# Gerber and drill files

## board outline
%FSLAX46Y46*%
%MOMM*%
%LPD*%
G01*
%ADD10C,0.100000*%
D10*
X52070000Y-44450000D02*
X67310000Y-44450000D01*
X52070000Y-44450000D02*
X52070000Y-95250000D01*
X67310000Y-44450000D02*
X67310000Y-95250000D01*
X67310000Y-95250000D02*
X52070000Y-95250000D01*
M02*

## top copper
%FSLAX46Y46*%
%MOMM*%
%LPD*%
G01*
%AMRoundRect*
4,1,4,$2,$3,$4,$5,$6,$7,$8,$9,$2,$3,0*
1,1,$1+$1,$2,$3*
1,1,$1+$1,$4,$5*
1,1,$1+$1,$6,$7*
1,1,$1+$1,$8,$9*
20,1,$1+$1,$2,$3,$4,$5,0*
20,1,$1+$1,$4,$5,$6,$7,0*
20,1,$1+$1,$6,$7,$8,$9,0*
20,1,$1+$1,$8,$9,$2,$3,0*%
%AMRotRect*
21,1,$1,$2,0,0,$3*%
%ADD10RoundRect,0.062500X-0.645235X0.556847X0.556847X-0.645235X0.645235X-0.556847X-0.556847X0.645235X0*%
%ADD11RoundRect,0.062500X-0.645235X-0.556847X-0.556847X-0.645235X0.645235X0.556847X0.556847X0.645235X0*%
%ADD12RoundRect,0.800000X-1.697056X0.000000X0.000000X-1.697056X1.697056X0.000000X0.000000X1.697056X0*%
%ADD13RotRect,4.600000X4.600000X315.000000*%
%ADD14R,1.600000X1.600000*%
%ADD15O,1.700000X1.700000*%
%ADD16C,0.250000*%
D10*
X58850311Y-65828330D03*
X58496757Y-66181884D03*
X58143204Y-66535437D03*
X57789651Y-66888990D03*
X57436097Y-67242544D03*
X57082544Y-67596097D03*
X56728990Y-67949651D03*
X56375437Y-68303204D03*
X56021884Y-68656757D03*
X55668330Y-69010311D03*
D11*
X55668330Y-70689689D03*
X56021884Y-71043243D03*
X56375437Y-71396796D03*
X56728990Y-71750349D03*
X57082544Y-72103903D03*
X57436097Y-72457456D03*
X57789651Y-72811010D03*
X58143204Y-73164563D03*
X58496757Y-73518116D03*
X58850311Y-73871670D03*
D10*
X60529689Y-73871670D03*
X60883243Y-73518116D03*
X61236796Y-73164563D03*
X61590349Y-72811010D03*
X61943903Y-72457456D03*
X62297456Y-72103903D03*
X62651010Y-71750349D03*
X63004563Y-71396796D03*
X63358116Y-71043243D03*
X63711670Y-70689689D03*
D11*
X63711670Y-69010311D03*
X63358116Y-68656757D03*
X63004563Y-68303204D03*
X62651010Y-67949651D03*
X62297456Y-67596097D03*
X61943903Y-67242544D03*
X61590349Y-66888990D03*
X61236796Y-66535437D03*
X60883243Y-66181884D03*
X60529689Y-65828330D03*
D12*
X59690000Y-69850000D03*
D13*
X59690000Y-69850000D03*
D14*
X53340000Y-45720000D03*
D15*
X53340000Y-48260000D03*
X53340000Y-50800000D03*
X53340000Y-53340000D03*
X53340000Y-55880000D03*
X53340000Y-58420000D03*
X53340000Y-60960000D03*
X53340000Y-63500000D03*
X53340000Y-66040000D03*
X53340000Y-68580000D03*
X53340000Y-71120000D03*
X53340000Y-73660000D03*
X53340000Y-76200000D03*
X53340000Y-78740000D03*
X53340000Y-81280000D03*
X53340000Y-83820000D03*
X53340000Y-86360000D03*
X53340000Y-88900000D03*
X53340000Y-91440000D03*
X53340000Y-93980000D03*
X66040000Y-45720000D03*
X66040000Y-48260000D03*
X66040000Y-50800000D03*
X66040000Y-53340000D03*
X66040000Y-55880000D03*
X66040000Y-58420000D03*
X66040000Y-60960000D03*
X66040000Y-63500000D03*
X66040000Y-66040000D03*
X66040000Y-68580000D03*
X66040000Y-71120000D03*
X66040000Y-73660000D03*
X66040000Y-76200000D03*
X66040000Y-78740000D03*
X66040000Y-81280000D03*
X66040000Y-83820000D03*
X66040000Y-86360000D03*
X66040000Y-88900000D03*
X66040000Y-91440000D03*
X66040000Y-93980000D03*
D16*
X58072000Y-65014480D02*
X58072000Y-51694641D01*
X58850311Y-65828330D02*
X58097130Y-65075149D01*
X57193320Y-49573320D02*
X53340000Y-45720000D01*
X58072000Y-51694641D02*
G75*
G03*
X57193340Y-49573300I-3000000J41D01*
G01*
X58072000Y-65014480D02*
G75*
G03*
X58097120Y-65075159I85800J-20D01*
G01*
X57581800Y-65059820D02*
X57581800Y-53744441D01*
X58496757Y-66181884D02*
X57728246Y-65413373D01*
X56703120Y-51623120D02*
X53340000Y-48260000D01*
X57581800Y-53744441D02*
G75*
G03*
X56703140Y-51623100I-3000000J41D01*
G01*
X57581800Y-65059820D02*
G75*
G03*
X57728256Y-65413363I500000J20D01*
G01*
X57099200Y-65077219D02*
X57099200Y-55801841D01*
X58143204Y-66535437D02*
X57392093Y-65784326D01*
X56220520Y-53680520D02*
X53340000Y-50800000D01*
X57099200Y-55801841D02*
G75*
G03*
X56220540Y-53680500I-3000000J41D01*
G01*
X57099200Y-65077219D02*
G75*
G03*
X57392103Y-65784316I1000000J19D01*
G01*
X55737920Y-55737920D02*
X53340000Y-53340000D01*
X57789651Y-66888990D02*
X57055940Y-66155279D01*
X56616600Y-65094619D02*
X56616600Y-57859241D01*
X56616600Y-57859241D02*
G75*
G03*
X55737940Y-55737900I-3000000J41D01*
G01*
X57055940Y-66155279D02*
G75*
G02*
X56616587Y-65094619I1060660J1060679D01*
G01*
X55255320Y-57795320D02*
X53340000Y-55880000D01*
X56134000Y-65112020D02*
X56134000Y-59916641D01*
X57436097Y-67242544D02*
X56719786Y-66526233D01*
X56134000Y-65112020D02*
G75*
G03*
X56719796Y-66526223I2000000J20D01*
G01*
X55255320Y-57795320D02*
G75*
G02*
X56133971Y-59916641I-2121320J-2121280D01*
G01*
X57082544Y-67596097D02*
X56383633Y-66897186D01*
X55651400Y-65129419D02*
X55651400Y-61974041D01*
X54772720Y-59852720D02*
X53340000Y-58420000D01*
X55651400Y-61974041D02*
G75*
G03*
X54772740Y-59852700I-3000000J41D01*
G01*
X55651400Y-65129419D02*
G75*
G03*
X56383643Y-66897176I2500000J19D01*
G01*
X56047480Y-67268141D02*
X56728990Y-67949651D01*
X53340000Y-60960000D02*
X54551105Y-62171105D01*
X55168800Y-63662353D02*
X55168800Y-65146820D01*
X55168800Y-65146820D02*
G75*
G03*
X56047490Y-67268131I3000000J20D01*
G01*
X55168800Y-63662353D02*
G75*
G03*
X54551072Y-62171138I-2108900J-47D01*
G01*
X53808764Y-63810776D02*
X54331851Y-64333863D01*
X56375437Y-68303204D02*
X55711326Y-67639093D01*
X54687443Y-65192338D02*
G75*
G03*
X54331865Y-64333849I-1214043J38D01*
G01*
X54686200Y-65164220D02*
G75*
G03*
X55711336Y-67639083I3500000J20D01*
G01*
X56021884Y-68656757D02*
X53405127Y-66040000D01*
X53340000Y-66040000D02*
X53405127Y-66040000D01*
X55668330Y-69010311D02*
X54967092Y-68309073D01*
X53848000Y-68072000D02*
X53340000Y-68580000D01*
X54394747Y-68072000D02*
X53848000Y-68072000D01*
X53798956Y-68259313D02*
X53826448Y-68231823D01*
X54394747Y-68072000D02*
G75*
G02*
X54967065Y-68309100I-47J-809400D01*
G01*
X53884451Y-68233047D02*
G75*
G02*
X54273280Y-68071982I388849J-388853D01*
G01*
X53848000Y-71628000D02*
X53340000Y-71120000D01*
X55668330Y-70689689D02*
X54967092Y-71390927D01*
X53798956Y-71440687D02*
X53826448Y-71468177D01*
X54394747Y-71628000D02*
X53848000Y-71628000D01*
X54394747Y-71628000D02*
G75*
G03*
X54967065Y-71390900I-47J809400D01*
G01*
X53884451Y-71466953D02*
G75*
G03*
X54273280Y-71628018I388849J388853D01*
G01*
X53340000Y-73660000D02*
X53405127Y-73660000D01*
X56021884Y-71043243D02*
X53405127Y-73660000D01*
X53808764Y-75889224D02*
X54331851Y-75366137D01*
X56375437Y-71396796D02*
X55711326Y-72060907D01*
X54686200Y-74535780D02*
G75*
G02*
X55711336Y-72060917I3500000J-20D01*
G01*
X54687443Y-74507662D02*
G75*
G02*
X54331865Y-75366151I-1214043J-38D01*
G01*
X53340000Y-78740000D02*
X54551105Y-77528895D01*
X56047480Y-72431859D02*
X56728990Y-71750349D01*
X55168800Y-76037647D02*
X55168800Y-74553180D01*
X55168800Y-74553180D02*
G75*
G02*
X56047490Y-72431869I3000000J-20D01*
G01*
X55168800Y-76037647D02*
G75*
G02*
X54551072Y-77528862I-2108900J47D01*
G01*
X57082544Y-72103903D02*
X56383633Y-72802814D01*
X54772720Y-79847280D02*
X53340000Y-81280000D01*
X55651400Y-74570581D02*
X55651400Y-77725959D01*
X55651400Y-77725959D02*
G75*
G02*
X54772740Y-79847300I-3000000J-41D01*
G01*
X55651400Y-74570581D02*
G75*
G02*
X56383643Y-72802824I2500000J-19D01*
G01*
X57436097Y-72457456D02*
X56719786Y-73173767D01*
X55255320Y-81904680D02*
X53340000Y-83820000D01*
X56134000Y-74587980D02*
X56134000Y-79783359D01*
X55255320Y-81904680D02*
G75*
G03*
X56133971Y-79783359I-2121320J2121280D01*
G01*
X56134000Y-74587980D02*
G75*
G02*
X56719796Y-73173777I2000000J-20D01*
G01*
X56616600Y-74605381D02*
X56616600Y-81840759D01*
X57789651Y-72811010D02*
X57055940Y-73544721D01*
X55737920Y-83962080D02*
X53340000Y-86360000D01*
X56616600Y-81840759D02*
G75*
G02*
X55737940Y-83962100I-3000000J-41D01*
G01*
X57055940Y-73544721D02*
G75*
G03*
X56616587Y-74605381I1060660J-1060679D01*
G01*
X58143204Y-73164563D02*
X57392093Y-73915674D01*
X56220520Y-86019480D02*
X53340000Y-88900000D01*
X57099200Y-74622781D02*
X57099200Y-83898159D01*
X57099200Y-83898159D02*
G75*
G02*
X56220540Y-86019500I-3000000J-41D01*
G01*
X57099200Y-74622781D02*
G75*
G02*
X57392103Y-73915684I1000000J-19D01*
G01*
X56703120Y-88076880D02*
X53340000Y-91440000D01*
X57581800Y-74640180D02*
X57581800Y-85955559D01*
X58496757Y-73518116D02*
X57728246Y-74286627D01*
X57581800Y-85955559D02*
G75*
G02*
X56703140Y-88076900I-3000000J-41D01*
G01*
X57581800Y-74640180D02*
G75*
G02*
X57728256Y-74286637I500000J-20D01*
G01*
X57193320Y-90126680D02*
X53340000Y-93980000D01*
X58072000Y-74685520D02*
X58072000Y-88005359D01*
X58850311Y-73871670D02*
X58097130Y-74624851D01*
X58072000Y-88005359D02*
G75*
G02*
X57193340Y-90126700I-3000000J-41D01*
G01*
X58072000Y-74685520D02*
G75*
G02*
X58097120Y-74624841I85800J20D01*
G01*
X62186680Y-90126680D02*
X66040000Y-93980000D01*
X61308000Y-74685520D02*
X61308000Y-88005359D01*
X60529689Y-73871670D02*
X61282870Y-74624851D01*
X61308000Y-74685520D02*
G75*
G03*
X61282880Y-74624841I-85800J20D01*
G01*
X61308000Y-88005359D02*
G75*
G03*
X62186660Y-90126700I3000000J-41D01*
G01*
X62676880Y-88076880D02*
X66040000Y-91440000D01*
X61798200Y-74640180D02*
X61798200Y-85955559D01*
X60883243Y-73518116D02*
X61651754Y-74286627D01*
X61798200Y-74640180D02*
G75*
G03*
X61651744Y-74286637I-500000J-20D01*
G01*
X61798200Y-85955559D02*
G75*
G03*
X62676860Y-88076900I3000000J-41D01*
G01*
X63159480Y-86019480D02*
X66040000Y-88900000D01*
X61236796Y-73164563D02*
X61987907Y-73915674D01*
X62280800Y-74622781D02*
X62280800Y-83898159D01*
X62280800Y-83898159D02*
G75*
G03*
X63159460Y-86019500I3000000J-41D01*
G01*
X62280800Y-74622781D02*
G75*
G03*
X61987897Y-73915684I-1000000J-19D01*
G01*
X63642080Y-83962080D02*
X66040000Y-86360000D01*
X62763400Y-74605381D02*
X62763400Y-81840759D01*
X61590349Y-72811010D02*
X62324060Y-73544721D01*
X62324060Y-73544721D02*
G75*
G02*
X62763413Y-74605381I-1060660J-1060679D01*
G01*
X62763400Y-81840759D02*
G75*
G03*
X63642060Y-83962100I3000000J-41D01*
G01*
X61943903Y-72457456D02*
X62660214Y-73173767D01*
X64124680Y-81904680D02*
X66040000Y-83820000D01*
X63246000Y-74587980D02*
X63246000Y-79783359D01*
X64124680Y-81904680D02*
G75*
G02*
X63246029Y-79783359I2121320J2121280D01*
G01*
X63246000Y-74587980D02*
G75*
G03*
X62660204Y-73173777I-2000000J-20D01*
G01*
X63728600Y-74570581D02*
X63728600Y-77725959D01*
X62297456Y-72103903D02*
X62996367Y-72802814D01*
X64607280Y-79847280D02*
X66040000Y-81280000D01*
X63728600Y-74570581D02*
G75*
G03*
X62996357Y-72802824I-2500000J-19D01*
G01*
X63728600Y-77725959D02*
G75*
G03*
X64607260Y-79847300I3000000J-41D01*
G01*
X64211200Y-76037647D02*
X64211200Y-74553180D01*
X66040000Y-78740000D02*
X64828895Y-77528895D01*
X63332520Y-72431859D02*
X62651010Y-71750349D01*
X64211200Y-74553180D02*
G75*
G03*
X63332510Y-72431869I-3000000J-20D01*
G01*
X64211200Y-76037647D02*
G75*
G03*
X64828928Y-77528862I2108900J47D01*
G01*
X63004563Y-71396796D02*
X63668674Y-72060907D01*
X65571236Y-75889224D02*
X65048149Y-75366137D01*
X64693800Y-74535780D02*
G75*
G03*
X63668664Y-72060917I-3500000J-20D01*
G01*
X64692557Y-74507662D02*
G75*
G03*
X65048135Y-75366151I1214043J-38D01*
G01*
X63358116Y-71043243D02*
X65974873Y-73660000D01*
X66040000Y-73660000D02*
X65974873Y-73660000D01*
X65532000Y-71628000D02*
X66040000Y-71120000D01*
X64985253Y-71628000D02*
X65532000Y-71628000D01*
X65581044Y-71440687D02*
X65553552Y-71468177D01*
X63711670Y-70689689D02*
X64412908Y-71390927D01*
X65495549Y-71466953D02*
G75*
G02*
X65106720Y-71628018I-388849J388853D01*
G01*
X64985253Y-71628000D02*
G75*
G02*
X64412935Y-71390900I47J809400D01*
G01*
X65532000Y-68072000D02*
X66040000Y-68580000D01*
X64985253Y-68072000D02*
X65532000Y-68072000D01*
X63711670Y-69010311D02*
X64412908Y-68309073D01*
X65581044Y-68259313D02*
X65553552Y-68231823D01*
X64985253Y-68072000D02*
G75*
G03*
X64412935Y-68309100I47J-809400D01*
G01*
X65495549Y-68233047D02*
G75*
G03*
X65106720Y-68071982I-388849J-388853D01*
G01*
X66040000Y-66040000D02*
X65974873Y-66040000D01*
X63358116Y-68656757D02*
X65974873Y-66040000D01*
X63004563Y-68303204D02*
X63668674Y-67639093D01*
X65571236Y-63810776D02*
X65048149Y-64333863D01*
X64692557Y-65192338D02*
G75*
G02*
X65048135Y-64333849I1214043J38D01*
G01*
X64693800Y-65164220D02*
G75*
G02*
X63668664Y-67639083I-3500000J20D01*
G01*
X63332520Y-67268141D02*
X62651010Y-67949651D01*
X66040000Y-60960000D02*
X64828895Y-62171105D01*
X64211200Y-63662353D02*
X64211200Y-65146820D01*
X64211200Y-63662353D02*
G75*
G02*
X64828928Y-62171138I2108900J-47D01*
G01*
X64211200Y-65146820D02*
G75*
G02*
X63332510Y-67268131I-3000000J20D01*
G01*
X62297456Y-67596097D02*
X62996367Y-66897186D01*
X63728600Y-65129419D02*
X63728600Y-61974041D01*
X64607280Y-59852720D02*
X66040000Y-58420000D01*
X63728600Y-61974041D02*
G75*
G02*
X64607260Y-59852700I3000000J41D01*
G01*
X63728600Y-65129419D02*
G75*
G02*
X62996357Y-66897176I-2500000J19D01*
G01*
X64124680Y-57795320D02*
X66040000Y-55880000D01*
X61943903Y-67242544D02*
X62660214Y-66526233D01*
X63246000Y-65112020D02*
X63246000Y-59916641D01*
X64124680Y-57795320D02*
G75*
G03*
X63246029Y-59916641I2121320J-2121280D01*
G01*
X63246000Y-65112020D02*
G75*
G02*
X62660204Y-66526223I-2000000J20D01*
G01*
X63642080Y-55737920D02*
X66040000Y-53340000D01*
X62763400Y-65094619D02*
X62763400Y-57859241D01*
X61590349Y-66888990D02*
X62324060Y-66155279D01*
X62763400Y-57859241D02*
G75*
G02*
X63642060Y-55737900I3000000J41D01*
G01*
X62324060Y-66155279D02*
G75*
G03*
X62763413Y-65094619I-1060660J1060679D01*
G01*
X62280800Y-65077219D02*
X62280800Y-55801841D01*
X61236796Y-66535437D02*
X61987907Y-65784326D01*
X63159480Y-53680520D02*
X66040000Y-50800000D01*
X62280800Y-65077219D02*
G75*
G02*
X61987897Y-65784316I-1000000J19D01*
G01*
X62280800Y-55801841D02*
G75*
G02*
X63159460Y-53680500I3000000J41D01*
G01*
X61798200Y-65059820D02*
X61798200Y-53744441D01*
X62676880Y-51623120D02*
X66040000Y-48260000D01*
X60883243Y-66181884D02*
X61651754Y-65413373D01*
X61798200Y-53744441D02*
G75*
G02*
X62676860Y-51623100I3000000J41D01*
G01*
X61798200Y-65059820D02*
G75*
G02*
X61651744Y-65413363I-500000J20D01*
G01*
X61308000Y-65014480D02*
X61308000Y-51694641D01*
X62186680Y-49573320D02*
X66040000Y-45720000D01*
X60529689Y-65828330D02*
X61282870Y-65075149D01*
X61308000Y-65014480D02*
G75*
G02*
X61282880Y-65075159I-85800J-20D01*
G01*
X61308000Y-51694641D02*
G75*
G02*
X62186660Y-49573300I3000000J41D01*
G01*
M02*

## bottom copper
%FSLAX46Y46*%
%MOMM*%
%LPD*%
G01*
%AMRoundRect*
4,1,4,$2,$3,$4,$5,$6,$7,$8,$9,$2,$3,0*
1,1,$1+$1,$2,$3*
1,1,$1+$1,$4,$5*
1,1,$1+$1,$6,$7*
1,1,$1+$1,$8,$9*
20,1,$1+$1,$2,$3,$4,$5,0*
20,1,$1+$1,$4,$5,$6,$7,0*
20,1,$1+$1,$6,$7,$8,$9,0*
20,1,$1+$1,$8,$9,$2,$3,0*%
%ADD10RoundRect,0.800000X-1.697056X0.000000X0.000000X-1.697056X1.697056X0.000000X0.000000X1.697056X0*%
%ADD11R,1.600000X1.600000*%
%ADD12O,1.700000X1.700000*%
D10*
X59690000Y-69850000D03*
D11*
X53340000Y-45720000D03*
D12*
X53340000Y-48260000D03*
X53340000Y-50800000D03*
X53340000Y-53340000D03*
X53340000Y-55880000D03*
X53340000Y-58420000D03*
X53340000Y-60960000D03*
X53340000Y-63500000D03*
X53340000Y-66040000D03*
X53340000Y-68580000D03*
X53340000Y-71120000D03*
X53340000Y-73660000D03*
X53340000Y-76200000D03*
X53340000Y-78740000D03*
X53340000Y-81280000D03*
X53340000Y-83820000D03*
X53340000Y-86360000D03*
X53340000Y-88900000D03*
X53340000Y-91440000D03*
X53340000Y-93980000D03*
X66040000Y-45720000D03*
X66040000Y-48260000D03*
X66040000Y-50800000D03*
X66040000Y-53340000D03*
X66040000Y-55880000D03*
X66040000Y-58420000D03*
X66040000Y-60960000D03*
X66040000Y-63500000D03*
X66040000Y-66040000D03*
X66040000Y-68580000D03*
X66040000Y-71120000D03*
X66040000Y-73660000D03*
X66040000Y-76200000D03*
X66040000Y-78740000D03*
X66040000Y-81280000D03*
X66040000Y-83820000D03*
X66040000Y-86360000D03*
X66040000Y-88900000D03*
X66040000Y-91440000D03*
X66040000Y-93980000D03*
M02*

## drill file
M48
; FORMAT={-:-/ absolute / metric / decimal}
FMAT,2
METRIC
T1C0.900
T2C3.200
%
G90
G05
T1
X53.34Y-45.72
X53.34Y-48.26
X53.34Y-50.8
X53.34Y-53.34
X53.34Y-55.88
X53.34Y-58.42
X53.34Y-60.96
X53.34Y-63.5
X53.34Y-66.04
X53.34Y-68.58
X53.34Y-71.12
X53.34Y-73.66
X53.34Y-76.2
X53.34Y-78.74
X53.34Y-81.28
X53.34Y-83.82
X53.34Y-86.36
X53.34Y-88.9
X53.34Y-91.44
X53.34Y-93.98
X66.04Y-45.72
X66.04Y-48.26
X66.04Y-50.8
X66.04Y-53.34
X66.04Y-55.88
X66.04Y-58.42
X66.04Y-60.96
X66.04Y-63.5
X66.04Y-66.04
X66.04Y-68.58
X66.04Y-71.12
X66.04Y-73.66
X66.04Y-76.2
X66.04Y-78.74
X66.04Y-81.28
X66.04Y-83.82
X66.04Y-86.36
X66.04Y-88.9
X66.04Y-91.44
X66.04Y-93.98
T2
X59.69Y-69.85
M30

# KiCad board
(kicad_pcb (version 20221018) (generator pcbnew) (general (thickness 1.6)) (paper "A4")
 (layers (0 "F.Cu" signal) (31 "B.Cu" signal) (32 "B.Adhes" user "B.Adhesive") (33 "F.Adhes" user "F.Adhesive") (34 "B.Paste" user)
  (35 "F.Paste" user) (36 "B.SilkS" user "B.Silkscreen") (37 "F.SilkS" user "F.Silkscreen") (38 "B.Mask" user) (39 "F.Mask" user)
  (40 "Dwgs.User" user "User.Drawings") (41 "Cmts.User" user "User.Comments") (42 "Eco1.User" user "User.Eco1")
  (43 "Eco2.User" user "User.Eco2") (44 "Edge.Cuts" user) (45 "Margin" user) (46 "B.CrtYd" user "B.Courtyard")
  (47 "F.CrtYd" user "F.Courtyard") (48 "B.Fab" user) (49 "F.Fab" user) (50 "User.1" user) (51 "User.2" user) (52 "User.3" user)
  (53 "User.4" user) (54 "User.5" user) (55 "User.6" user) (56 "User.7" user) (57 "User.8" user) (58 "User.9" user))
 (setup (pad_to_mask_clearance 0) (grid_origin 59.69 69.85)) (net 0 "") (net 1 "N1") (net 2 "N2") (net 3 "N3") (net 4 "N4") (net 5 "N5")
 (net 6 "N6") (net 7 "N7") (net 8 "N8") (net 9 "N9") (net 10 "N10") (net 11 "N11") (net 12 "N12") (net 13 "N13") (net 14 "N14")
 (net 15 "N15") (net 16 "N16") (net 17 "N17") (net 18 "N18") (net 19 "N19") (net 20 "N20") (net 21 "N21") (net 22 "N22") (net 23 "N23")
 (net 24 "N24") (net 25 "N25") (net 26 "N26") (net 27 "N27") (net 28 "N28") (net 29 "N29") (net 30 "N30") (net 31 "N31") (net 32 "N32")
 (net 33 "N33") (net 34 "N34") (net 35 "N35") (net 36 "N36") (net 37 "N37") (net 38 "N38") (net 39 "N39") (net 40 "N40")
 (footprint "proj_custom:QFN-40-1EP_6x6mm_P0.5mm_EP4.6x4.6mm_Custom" (layer "F.Cu") (at 59.69 69.85 -45)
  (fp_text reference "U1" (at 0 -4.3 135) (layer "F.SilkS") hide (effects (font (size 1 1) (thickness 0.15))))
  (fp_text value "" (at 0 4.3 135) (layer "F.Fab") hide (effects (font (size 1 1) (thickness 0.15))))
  (pad "" smd roundrect (at -1.725 -1.725 315) (size 0.93 0.93) (layers "F.Paste") (roundrect_rratio 0.25))
  (pad "" smd roundrect (at -1.725 -0.575 315) (size 0.93 0.93) (layers "F.Paste") (roundrect_rratio 0.25))
  (pad "" smd roundrect (at -1.725 0.575 315) (size 0.93 0.93) (layers "F.Paste") (roundrect_rratio 0.25))
  (pad "" smd roundrect (at -1.725 1.725 315) (size 0.93 0.93) (layers "F.Paste") (roundrect_rratio 0.25))
  (pad "" smd roundrect (at -0.575 -1.725 315) (size 0.93 0.93) (layers "F.Paste") (roundrect_rratio 0.25))
  (pad "" smd roundrect (at -0.575 -0.575 315) (size 0.93 0.93) (layers "F.Paste") (roundrect_rratio 0.25))
  (pad "" smd roundrect (at -0.575 0.575 315) (size 0.93 0.93) (layers "F.Paste") (roundrect_rratio 0.25))
  (pad "" smd roundrect (at -0.575 1.725 315) (size 0.93 0.93) (layers "F.Paste") (roundrect_rratio 0.25))
  (pad "" smd roundrect (at 0.575 -1.725 315) (size 0.93 0.93) (layers "F.Paste") (roundrect_rratio 0.25))
  (pad "" smd roundrect (at 0.575 -0.575 315) (size 0.93 0.93) (layers "F.Paste") (roundrect_rratio 0.25))
  (pad "" smd roundrect (at 0.575 0.575 315) (size 0.93 0.93) (layers "F.Paste") (roundrect_rratio 0.25))
  (pad "" smd roundrect (at 0.575 1.725 315) (size 0.93 0.93) (layers "F.Paste") (roundrect_rratio 0.25))
  (pad "" smd roundrect (at 1.725 -1.725 315) (size 0.93 0.93) (layers "F.Paste") (roundrect_rratio 0.25))
  (pad "" smd roundrect (at 1.725 -0.575 315) (size 0.93 0.93) (layers "F.Paste") (roundrect_rratio 0.25))
  (pad "" smd roundrect (at 1.725 0.575 315) (size 0.93 0.93) (layers "F.Paste") (roundrect_rratio 0.25))
  (pad "" smd roundrect (at 1.725 1.725 315) (size 0.93 0.93) (layers "F.Paste") (roundrect_rratio 0.25))
  (pad "1" smd roundrect (at -3.4375 -2.25 315) (size 1.825 0.25) (layers "F.Cu" "F.Paste" "F.Mask") (roundrect_rratio 0.25) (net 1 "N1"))
  (pad "2" smd roundrect (at -3.4375 -1.75 315) (size 1.825 0.25) (layers "F.Cu" "F.Paste" "F.Mask") (roundrect_rratio 0.25) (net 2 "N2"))
  (pad "3" smd roundrect (at -3.4375 -1.25 315) (size 1.825 0.25) (layers "F.Cu" "F.Paste" "F.Mask") (roundrect_rratio 0.25) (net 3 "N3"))
  (pad "4" smd roundrect (at -3.4375 -0.75 315) (size 1.825 0.25) (layers "F.Cu" "F.Paste" "F.Mask") (roundrect_rratio 0.25) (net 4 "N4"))
  (pad "5" smd roundrect (at -3.4375 -0.25 315) (size 1.825 0.25) (layers "F.Cu" "F.Paste" "F.Mask") (roundrect_rratio 0.25) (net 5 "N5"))
  (pad "6" smd roundrect (at -3.4375 0.25 315) (size 1.825 0.25) (layers "F.Cu" "F.Paste" "F.Mask") (roundrect_rratio 0.25) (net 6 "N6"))
  (pad "7" smd roundrect (at -3.4375 0.75 315) (size 1.825 0.25) (layers "F.Cu" "F.Paste" "F.Mask") (roundrect_rratio 0.25) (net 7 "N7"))
  (pad "8" smd roundrect (at -3.4375 1.25 315) (size 1.825 0.25) (layers "F.Cu" "F.Paste" "F.Mask") (roundrect_rratio 0.25) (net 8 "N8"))
  (pad "9" smd roundrect (at -3.4375 1.75 315) (size 1.825 0.25) (layers "F.Cu" "F.Paste" "F.Mask") (roundrect_rratio 0.25) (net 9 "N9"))
  (pad "10" smd roundrect (at -3.4375 2.25 315) (size 1.825 0.25) (layers "F.Cu" "F.Paste" "F.Mask") (roundrect_rratio 0.25) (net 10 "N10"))
  (pad "11" smd roundrect (at -2.25 3.4375 315) (size 0.25 1.825) (layers "F.Cu" "F.Paste" "F.Mask") (roundrect_rratio 0.25) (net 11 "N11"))
  (pad "12" smd roundrect (at -1.75 3.4375 315) (size 0.25 1.825) (layers "F.Cu" "F.Paste" "F.Mask") (roundrect_rratio 0.25) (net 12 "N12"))
  (pad "13" smd roundrect (at -1.25 3.4375 315) (size 0.25 1.825) (layers "F.Cu" "F.Paste" "F.Mask") (roundrect_rratio 0.25) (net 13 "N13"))
  (pad "14" smd roundrect (at -0.75 3.4375 315) (size 0.25 1.825) (layers "F.Cu" "F.Paste" "F.Mask") (roundrect_rratio 0.25) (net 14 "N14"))
  (pad "15" smd roundrect (at -0.25 3.4375 315) (size 0.25 1.825) (layers "F.Cu" "F.Paste" "F.Mask") (roundrect_rratio 0.25) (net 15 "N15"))
  (pad "16" smd roundrect (at 0.25 3.4375 315) (size 0.25 1.825) (layers "F.Cu" "F.Paste" "F.Mask") (roundrect_rratio 0.25) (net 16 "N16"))
  (pad "17" smd roundrect (at 0.75 3.4375 315) (size 0.25 1.825) (layers "F.Cu" "F.Paste" "F.Mask") (roundrect_rratio 0.25) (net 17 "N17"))
  (pad "18" smd roundrect (at 1.25 3.4375 315) (size 0.25 1.825) (layers "F.Cu" "F.Paste" "F.Mask") (roundrect_rratio 0.25) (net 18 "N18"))
  (pad "19" smd roundrect (at 1.75 3.4375 315) (size 0.25 1.825) (layers "F.Cu" "F.Paste" "F.Mask") (roundrect_rratio 0.25) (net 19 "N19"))
  (pad "20" smd roundrect (at 2.25 3.4375 315) (size 0.25 1.825) (layers "F.Cu" "F.Paste" "F.Mask") (roundrect_rratio 0.25) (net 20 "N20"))
  (pad "21" smd roundrect (at 3.4375 2.25 315) (size 1.825 0.25) (layers "F.Cu" "F.Paste" "F.Mask") (roundrect_rratio 0.25) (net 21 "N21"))
  (pad "22" smd roundrect (at 3.4375 1.75 315) (size 1.825 0.25) (layers "F.Cu" "F.Paste" "F.Mask") (roundrect_rratio 0.25) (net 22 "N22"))
  (pad "23" smd roundrect (at 3.4375 1.25 315) (size 1.825 0.25) (layers "F.Cu" "F.Paste" "F.Mask") (roundrect_rratio 0.25) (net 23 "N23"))
  (pad "24" smd roundrect (at 3.4375 0.75 315) (size 1.825 0.25) (layers "F.Cu" "F.Paste" "F.Mask") (roundrect_rratio 0.25) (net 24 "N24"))
  (pad "25" smd roundrect (at 3.4375 0.25 315) (size 1.825 0.25) (layers "F.Cu" "F.Paste" "F.Mask") (roundrect_rratio 0.25) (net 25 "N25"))
  (pad "26" smd roundrect (at 3.4375 -0.25 315) (size 1.825 0.25) (layers "F.Cu" "F.Paste" "F.Mask") (roundrect_rratio 0.25) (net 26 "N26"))
  (pad "27" smd roundrect (at 3.4375 -0.75 315) (size 1.825 0.25) (layers "F.Cu" "F.Paste" "F.Mask") (roundrect_rratio 0.25) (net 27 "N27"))
  (pad "28" smd roundrect (at 3.4375 -1.25 315) (size 1.825 0.25) (layers "F.Cu" "F.Paste" "F.Mask") (roundrect_rratio 0.25) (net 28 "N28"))
  (pad "29" smd roundrect (at 3.4375 -1.75 315) (size 1.825 0.25) (layers "F.Cu" "F.Paste" "F.Mask") (roundrect_rratio 0.25) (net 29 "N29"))
  (pad "30" smd roundrect (at 3.4375 -2.25 315) (size 1.825 0.25) (layers "F.Cu" "F.Paste" "F.Mask") (roundrect_rratio 0.25) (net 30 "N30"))
  (pad "31" smd roundrect (at 2.25 -3.4375 315) (size 0.25 1.825) (layers "F.Cu" "F.Paste" "F.Mask") (roundrect_rratio 0.25) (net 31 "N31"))
  (pad "32" smd roundrect (at 1.75 -3.4375 315) (size 0.25 1.825) (layers "F.Cu" "F.Paste" "F.Mask") (roundrect_rratio 0.25) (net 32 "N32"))
  (pad "33" smd roundrect (at 1.25 -3.4375 315) (size 0.25 1.825) (layers "F.Cu" "F.Paste" "F.Mask") (roundrect_rratio 0.25) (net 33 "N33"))
  (pad "34" smd roundrect (at 0.75 -3.4375 315) (size 0.25 1.825) (layers "F.Cu" "F.Paste" "F.Mask") (roundrect_rratio 0.25) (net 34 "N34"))
  (pad "35" smd roundrect (at 0.25 -3.4375 315) (size 0.25 1.825) (layers "F.Cu" "F.Paste" "F.Mask") (roundrect_rratio 0.25) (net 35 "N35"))
  (pad "36" smd roundrect (at -0.25 -3.4375 315) (size 0.25 1.825) (layers "F.Cu" "F.Paste" "F.Mask") (roundrect_rratio 0.25) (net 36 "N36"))
  (pad "37" smd roundrect (at -0.75 -3.4375 315) (size 0.25 1.825) (layers "F.Cu" "F.Paste" "F.Mask") (roundrect_rratio 0.25) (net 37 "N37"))
  (pad "38" smd roundrect (at -1.25 -3.4375 315) (size 0.25 1.825) (layers "F.Cu" "F.Paste" "F.Mask") (roundrect_rratio 0.25) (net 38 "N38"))
  (pad "39" smd roundrect (at -1.75 -3.4375 315) (size 0.25 1.825) (layers "F.Cu" "F.Paste" "F.Mask") (roundrect_rratio 0.25) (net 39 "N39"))
  (pad "40" smd roundrect (at -2.25 -3.4375 315) (size 0.25 1.825) (layers "F.Cu" "F.Paste" "F.Mask") (roundrect_rratio 0.25) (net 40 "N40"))
  (pad "41" thru_hole roundrect (at 0 0 315) (size 4 4) (drill 3.2) (layers "*.Cu" "*.Mask") (roundrect_rratio 0.2)
   (thermal_bridge_angle 45))
  (pad "41" smd rect (at 0 0 315) (size 4.6 4.6) (layers "F.Cu" "F.Mask")))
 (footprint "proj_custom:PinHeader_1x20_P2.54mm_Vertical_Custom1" (layer "B.Cu") (at 53.34 45.72 180)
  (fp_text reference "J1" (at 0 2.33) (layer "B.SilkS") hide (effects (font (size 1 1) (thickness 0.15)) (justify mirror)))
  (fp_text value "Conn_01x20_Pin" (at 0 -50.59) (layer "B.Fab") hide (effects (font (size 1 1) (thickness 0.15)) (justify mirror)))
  (pad "1" thru_hole rect (at 0 0 180) (size 1.6 1.6) (drill 0.9) (layers "*.Cu" "*.Mask") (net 1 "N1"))
  (pad "2" thru_hole oval (at 0 -2.54 180) (size 1.7 1.7) (drill 0.9) (layers "*.Cu" "*.Mask") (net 2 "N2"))
  (pad "3" thru_hole oval (at 0 -5.08 180) (size 1.7 1.7) (drill 0.9) (layers "*.Cu" "*.Mask") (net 3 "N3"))
  (pad "4" thru_hole oval (at 0 -7.62 180) (size 1.7 1.7) (drill 0.9) (layers "*.Cu" "*.Mask") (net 4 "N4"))
  (pad "5" thru_hole oval (at 0 -10.16 180) (size 1.7 1.7) (drill 0.9) (layers "*.Cu" "*.Mask") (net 5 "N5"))
  (pad "6" thru_hole oval (at 0 -12.7 180) (size 1.7 1.7) (drill 0.9) (layers "*.Cu" "*.Mask") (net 6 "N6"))
  (pad "7" thru_hole oval (at 0 -15.24 180) (size 1.7 1.7) (drill 0.9) (layers "*.Cu" "*.Mask") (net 7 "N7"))
  (pad "8" thru_hole oval (at 0 -17.78 180) (size 1.7 1.7) (drill 0.9) (layers "*.Cu" "*.Mask") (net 8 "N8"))
  (pad "9" thru_hole oval (at 0 -20.32 180) (size 1.7 1.7) (drill 0.9) (layers "*.Cu" "*.Mask") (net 9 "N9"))
  (pad "10" thru_hole oval (at 0 -22.86 180) (size 1.7 1.7) (drill 0.9) (layers "*.Cu" "*.Mask") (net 10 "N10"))
  (pad "11" thru_hole oval (at 0 -25.4 180) (size 1.7 1.7) (drill 0.9) (layers "*.Cu" "*.Mask") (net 11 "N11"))
  (pad "12" thru_hole oval (at 0 -27.94 180) (size 1.7 1.7) (drill 0.9) (layers "*.Cu" "*.Mask") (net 12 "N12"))
  (pad "13" thru_hole oval (at 0 -30.48 180) (size 1.7 1.7) (drill 0.9) (layers "*.Cu" "*.Mask") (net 13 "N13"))
  (pad "14" thru_hole oval (at 0 -33.02 180) (size 1.7 1.7) (drill 0.9) (layers "*.Cu" "*.Mask") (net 14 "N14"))
  (pad "15" thru_hole oval (at 0 -35.56 180) (size 1.7 1.7) (drill 0.9) (layers "*.Cu" "*.Mask") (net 15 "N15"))
  (pad "16" thru_hole oval (at 0 -38.1 180) (size 1.7 1.7) (drill 0.9) (layers "*.Cu" "*.Mask") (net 16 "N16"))
  (pad "17" thru_hole oval (at 0 -40.64 180) (size 1.7 1.7) (drill 0.9) (layers "*.Cu" "*.Mask") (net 17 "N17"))
  (pad "18" thru_hole oval (at 0 -43.18 180) (size 1.7 1.7) (drill 0.9) (layers "*.Cu" "*.Mask") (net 18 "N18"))
  (pad "19" thru_hole oval (at 0 -45.72 180) (size 1.7 1.7) (drill 0.9) (layers "*.Cu" "*.Mask") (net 19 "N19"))
  (pad "20" thru_hole oval (at 0 -48.26 180) (size 1.7 1.7) (drill 0.9) (layers "*.Cu" "*.Mask") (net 20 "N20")))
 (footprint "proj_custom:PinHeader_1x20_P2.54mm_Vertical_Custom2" (layer "B.Cu") (at 66.04 45.72 180)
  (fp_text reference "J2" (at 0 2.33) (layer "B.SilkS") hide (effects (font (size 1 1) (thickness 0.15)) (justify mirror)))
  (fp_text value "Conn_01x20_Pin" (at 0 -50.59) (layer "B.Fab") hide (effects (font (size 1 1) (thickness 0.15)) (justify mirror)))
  (pad "1" thru_hole oval (at 0 0 180) (size 1.7 1.7) (drill 0.9) (layers "*.Cu" "*.Mask") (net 40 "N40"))
  (pad "2" thru_hole oval (at 0 -2.54 180) (size 1.7 1.7) (drill 0.9) (layers "*.Cu" "*.Mask") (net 39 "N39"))
  (pad "3" thru_hole oval (at 0 -5.08 180) (size 1.7 1.7) (drill 0.9) (layers "*.Cu" "*.Mask") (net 38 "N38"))
  (pad "4" thru_hole oval (at 0 -7.62 180) (size 1.7 1.7) (drill 0.9) (layers "*.Cu" "*.Mask") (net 37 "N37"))
  (pad "5" thru_hole oval (at 0 -10.16 180) (size 1.7 1.7) (drill 0.9) (layers "*.Cu" "*.Mask") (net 36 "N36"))
  (pad "6" thru_hole oval (at 0 -12.7 180) (size 1.7 1.7) (drill 0.9) (layers "*.Cu" "*.Mask") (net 35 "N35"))
  (pad "7" thru_hole oval (at 0 -15.24 180) (size 1.7 1.7) (drill 0.9) (layers "*.Cu" "*.Mask") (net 34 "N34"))
  (pad "8" thru_hole oval (at 0 -17.78 180) (size 1.7 1.7) (drill 0.9) (layers "*.Cu" "*.Mask") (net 33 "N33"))
  (pad "9" thru_hole oval (at 0 -20.32 180) (size 1.7 1.7) (drill 0.9) (layers "*.Cu" "*.Mask") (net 32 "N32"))
  (pad "10" thru_hole oval (at 0 -22.86 180) (size 1.7 1.7) (drill 0.9) (layers "*.Cu" "*.Mask") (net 31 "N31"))
  (pad "11" thru_hole oval (at 0 -25.4 180) (size 1.7 1.7) (drill 0.9) (layers "*.Cu" "*.Mask") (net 30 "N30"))
  (pad "12" thru_hole oval (at 0 -27.94 180) (size 1.7 1.7) (drill 0.9) (layers "*.Cu" "*.Mask") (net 29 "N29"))
  (pad "13" thru_hole oval (at 0 -30.48 180) (size 1.7 1.7) (drill 0.9) (layers "*.Cu" "*.Mask") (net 28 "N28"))
  (pad "14" thru_hole oval (at 0 -33.02 180) (size 1.7 1.7) (drill 0.9) (layers "*.Cu" "*.Mask") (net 27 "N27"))
  (pad "15" thru_hole oval (at 0 -35.56 180) (size 1.7 1.7) (drill 0.9) (layers "*.Cu" "*.Mask") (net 26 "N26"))
  (pad "16" thru_hole oval (at 0 -38.1 180) (size 1.7 1.7) (drill 0.9) (layers "*.Cu" "*.Mask") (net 25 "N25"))
  (pad "17" thru_hole oval (at 0 -40.64 180) (size 1.7 1.7) (drill 0.9) (layers "*.Cu" "*.Mask") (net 24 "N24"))
  (pad "18" thru_hole oval (at 0 -43.18 180) (size 1.7 1.7) (drill 0.9) (layers "*.Cu" "*.Mask") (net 23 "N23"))
  (pad "19" thru_hole oval (at 0 -45.72 180) (size 1.7 1.7) (drill 0.9) (layers "*.Cu" "*.Mask") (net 22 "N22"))
  (pad "20" thru_hole oval (at 0 -48.26 180) (size 1.7 1.7) (drill 0.9) (layers "*.Cu" "*.Mask") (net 21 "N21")))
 (gr_line (start 52.07 44.45) (end 67.31 44.45) (stroke (width 0.1) (type default)) (layer "Edge.Cuts"))
 (gr_line (start 52.07 44.45) (end 52.07 95.25) (stroke (width 0.1) (type default)) (layer "Edge.Cuts"))
 (gr_line (start 67.31 44.45) (end 67.31 95.25) (stroke (width 0.1) (type default)) (layer "Edge.Cuts"))
 (gr_line (start 67.31 95.25) (end 52.07 95.25) (stroke (width 0.1) (type default)) (layer "Edge.Cuts"))
 (segment (start 58.072 65.01448) (end 58.072 51.694641) (width 0.25) (layer "F.Cu") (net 1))
 (segment (start 58.850311 65.82833) (end 58.09713 65.075149) (width 0.25) (layer "F.Cu") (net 1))
 (segment (start 57.19332 49.57332) (end 53.34 45.72) (width 0.25) (layer "F.Cu") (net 1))
 (arc (start 58.072 51.694641) (mid 57.843638 50.54659) (end 57.19332 49.57332) (width 0.25) (layer "F.Cu") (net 1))
 (arc (start 58.072 65.01448) (mid 58.078531 65.047314) (end 58.09713 65.075149) (width 0.25) (layer "F.Cu") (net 1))
 (segment (start 57.5818 65.05982) (end 57.5818 53.744441) (width 0.25) (layer "F.Cu") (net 2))
 (segment (start 58.496757 66.181884) (end 57.728246 65.413373) (width 0.25) (layer "F.Cu") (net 2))
 (segment (start 56.70312 51.62312) (end 53.34 48.26) (width 0.25) (layer "F.Cu") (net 2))
 (arc (start 57.5818 53.744441) (mid 57.353438 52.59639) (end 56.70312 51.62312) (width 0.25) (layer "F.Cu") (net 2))
 (arc (start 57.5818 65.05982) (mid 57.61986 65.251161) (end 57.728246 65.413373) (width 0.25) (layer "F.Cu") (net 2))
 (segment (start 57.0992 65.077219) (end 57.0992 55.801841) (width 0.25) (layer "F.Cu") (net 3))
 (segment (start 58.143204 66.535437) (end 57.392093 65.784326) (width 0.25) (layer "F.Cu") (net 3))
 (segment (start 56.22052 53.68052) (end 53.34 50.8) (width 0.25) (layer "F.Cu") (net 3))
 (arc (start 57.0992 55.801841) (mid 56.870838 54.65379) (end 56.22052 53.68052) (width 0.25) (layer "F.Cu") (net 3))
 (arc (start 57.0992 65.077219) (mid 57.17532 65.459902) (end 57.392093 65.784326) (width 0.25) (layer "F.Cu") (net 3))
 (segment (start 55.73792 55.73792) (end 53.34 53.34) (width 0.25) (layer "F.Cu") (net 4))
 (segment (start 57.789651 66.88899) (end 57.05594 66.155279) (width 0.25) (layer "F.Cu") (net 4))
 (segment (start 56.6166 65.094619) (end 56.6166 57.859241) (width 0.25) (layer "F.Cu") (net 4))
 (arc (start 56.6166 57.859241) (mid 56.388238 56.71119) (end 55.73792 55.73792) (width 0.25) (layer "F.Cu") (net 4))
 (arc (start 57.05594 66.155279) (mid 56.730781 65.668644) (end 56.6166 65.094619) (width 0.25) (layer "F.Cu") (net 4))
 (segment (start 55.25532 57.79532) (end 53.34 55.88) (width 0.25) (layer "F.Cu") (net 5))
 (segment (start 56.134 65.11202) (end 56.134 59.916641) (width 0.25) (layer "F.Cu") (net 5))
 (segment (start 57.436097 67.242544) (end 56.719786 66.526233) (width 0.25) (layer "F.Cu") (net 5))
 (arc (start 56.134 65.11202) (mid 56.286241 65.877387) (end 56.719786 66.526233) (width 0.25) (layer "F.Cu") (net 5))
 (arc (start 55.25532 57.79532) (mid 55.905639 58.76859) (end 56.134 59.916641) (width 0.25) (layer "F.Cu") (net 5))
 (segment (start 57.082544 67.596097) (end 56.383633 66.897186) (width 0.25) (layer "F.Cu") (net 6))
 (segment (start 55.6514 65.129419) (end 55.6514 61.974041) (width 0.25) (layer "F.Cu") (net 6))
 (segment (start 54.77272 59.85272) (end 53.34 58.42) (width 0.25) (layer "F.Cu") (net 6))
 (arc (start 55.6514 61.974041) (mid 55.423038 60.82599) (end 54.77272 59.85272) (width 0.25) (layer "F.Cu") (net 6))
 (arc (start 55.6514 65.129419) (mid 55.841701 66.086128) (end 56.383633 66.897186) (width 0.25) (layer "F.Cu") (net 6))
 (segment (start 56.04748 67.268141) (end 56.72899 67.949651) (width 0.25) (layer "F.Cu") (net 7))
 (segment (start 53.34 60.96) (end 54.551105 62.171105) (width 0.25) (layer "F.Cu") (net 7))
 (segment (start 55.1688 63.662353) (end 55.1688 65.14682) (width 0.25) (layer "F.Cu") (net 7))
 (arc (start 55.1688 65.14682) (mid 55.397162 66.294871) (end 56.04748 67.268141) (width 0.25) (layer "F.Cu") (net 7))
 (arc (start 55.1688 63.662353) (mid 55.008266 62.855295) (end 54.551105 62.171105) (width 0.25) (layer "F.Cu") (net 7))
 (segment (start 53.808764 63.810776) (end 54.331851 64.333863) (width 0.25) (layer "F.Cu") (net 8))
 (segment (start 56.375437 68.303204) (end 55.711326 67.639093) (width 0.25) (layer "F.Cu") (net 8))
 (arc (start 54.687443 65.192338) (mid 54.595028 64.727735) (end 54.331851 64.333863) (width 0.25) (layer "F.Cu") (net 8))
 (arc (start 54.6862 65.16422) (mid 54.952622 66.503612) (end 55.711326 67.639093) (width 0.25) (layer "F.Cu") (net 8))
 (segment (start 56.021884 68.656757) (end 53.405127 66.04) (width 0.25) (layer "F.Cu") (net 9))
 (segment (start 53.34 66.04) (end 53.405127 66.04) (width 0.25) (layer "F.Cu") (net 9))
 (segment (start 55.66833 69.010311) (end 54.967092 68.309073) (width 0.25) (layer "F.Cu") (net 10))
 (segment (start 53.848 68.072) (end 53.34 68.58) (width 0.25) (layer "F.Cu") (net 10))
 (segment (start 54.394747 68.072) (end 53.848 68.072) (width 0.25) (layer "F.Cu") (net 10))
 (segment (start 53.798956 68.259313) (end 53.826448 68.231823) (width 0.25) (layer "F.Cu") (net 10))
 (arc (start 54.394747 68.072) (mid 54.704498 68.133613) (end 54.967092 68.309073) (width 0.25) (layer "F.Cu") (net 10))
 (arc (start 53.884451 68.233047) (mid 54.062849 68.113854) (end 54.27328 68.072) (width 0.25) (layer "F.Cu") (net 10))
 (segment (start 53.848 71.628) (end 53.34 71.12) (width 0.25) (layer "F.Cu") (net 11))
 (segment (start 55.66833 70.689689) (end 54.967092 71.390927) (width 0.25) (layer "F.Cu") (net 11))
 (segment (start 53.798956 71.440687) (end 53.826448 71.468177) (width 0.25) (layer "F.Cu") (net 11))
 (segment (start 54.394747 71.628) (end 53.848 71.628) (width 0.25) (layer "F.Cu") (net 11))
 (arc (start 54.394747 71.628) (mid 54.704498 71.566387) (end 54.967092 71.390927) (width 0.25) (layer "F.Cu") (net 11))
 (arc (start 53.884451 71.466953) (mid 54.062849 71.586146) (end 54.27328 71.628) (width 0.25) (layer "F.Cu") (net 11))
 (segment (start 53.34 73.66) (end 53.405127 73.66) (width 0.25) (layer "F.Cu") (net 12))
 (segment (start 56.021884 71.043243) (end 53.405127 73.66) (width 0.25) (layer "F.Cu") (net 12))
 (segment (start 53.808764 75.889224) (end 54.331851 75.366137) (width 0.25) (layer "F.Cu") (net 13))
 (segment (start 56.375437 71.396796) (end 55.711326 72.060907) (width 0.25) (layer "F.Cu") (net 13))
 (arc (start 54.6862 74.53578) (mid 54.952622 73.196388) (end 55.711326 72.060907) (width 0.25) (layer "F.Cu") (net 13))
 (arc (start 54.687443 74.507662) (mid 54.595028 74.972265) (end 54.331851 75.366137) (width 0.25) (layer "F.Cu") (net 13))
 (segment (start 53.34 78.74) (end 54.551105 77.528895) (width 0.25) (layer "F.Cu") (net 14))
 (segment (start 56.04748 72.431859) (end 56.72899 71.750349) (width 0.25) (layer "F.Cu") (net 14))
 (segment (start 55.1688 76.037647) (end 55.1688 74.55318) (width 0.25) (layer "F.Cu") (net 14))
 (arc (start 55.1688 74.55318) (mid 55.397162 73.405129) (end 56.04748 72.431859) (width 0.25) (layer "F.Cu") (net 14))
 (arc (start 55.1688 76.037647) (mid 55.008266 76.844705) (end 54.551105 77.528895) (width 0.25) (layer "F.Cu") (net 14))
 (segment (start 57.082544 72.103903) (end 56.383633 72.802814) (width 0.25) (layer "F.Cu") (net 15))
 (segment (start 54.77272 79.84728) (end 53.34 81.28) (width 0.25) (layer "F.Cu") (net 15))
 (segment (start 55.6514 74.570581) (end 55.6514 77.725959) (width 0.25) (layer "F.Cu") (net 15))
 (arc (start 55.6514 77.725959) (mid 55.423038 78.87401) (end 54.77272 79.84728) (width 0.25) (layer "F.Cu") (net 15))
 (arc (start 55.6514 74.570581) (mid 55.841701 73.613872) (end 56.383633 72.802814) (width 0.25) (layer "F.Cu") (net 15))
 (segment (start 57.436097 72.457456) (end 56.719786 73.173767) (width 0.25) (layer "F.Cu") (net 16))
 (segment (start 55.25532 81.90468) (end 53.34 83.82) (width 0.25) (layer "F.Cu") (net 16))
 (segment (start 56.134 74.58798) (end 56.134 79.783359) (width 0.25) (layer "F.Cu") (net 16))
 (arc (start 55.25532 81.90468) (mid 55.905639 80.93141) (end 56.134 79.783359) (width 0.25) (layer "F.Cu") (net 16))
 (arc (start 56.134 74.58798) (mid 56.286241 73.822613) (end 56.719786 73.173767) (width 0.25) (layer "F.Cu") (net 16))
 (segment (start 56.6166 74.605381) (end 56.6166 81.840759) (width 0.25) (layer "F.Cu") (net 17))
 (segment (start 57.789651 72.81101) (end 57.05594 73.544721) (width 0.25) (layer "F.Cu") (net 17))
 (segment (start 55.73792 83.96208) (end 53.34 86.36) (width 0.25) (layer "F.Cu") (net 17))
 (arc (start 56.6166 81.840759) (mid 56.388238 82.98881) (end 55.73792 83.96208) (width 0.25) (layer "F.Cu") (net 17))
 (arc (start 57.05594 73.544721) (mid 56.730781 74.031356) (end 56.6166 74.605381) (width 0.25) (layer "F.Cu") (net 17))
 (segment (start 58.143204 73.164563) (end 57.392093 73.915674) (width 0.25) (layer "F.Cu") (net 18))
 (segment (start 56.22052 86.01948) (end 53.34 88.9) (width 0.25) (layer "F.Cu") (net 18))
 (segment (start 57.0992 74.622781) (end 57.0992 83.898159) (width 0.25) (layer "F.Cu") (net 18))
 (arc (start 57.0992 83.898159) (mid 56.870838 85.04621) (end 56.22052 86.01948) (width 0.25) (layer "F.Cu") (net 18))
 (arc (start 57.0992 74.622781) (mid 57.17532 74.240098) (end 57.392093 73.915674) (width 0.25) (layer "F.Cu") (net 18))
 (segment (start 56.70312 88.07688) (end 53.34 91.44) (width 0.25) (layer "F.Cu") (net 19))
 (segment (start 57.5818 74.64018) (end 57.5818 85.955559) (width 0.25) (layer "F.Cu") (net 19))
 (segment (start 58.496757 73.518116) (end 57.728246 74.286627) (width 0.25) (layer "F.Cu") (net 19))
 (arc (start 57.5818 85.955559) (mid 57.353438 87.10361) (end 56.70312 88.07688) (width 0.25) (layer "F.Cu") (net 19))
 (arc (start 57.5818 74.64018) (mid 57.61986 74.448839) (end 57.728246 74.286627) (width 0.25) (layer "F.Cu") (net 19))
 (segment (start 57.19332 90.12668) (end 53.34 93.98) (width 0.25) (layer "F.Cu") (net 20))
 (segment (start 58.072 74.68552) (end 58.072 88.005359) (width 0.25) (layer "F.Cu") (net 20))
 (segment (start 58.850311 73.87167) (end 58.09713 74.624851) (width 0.25) (layer "F.Cu") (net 20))
 (arc (start 58.072 88.005359) (mid 57.843638 89.15341) (end 57.19332 90.12668) (width 0.25) (layer "F.Cu") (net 20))
 (arc (start 58.072 74.68552) (mid 58.078531 74.652686) (end 58.09713 74.624851) (width 0.25) (layer "F.Cu") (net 20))
 (segment (start 62.18668 90.12668) (end 66.04 93.98) (width 0.25) (layer "F.Cu") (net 21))
 (segment (start 61.308 74.68552) (end 61.308 88.005359) (width 0.25) (layer "F.Cu") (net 21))
 (segment (start 60.529689 73.87167) (end 61.28287 74.624851) (width 0.25) (layer "F.Cu") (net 21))
 (arc (start 61.308 74.68552) (mid 61.301469 74.652686) (end 61.28287 74.624851) (width 0.25) (layer "F.Cu") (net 21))
 (arc (start 61.308 88.005359) (mid 61.536362 89.15341) (end 62.18668 90.12668) (width 0.25) (layer "F.Cu") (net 21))
 (segment (start 62.67688 88.07688) (end 66.04 91.44) (width 0.25) (layer "F.Cu") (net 22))
 (segment (start 61.7982 74.64018) (end 61.7982 85.955559) (width 0.25) (layer "F.Cu") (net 22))
 (segment (start 60.883243 73.518116) (end 61.651754 74.286627) (width 0.25) (layer "F.Cu") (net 22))
 (arc (start 61.7982 74.64018) (mid 61.76014 74.448839) (end 61.651754 74.286627) (width 0.25) (layer "F.Cu") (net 22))
 (arc (start 61.7982 85.955559) (mid 62.026562 87.10361) (end 62.67688 88.07688) (width 0.25) (layer "F.Cu") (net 22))
 (segment (start 63.15948 86.01948) (end 66.04 88.9) (width 0.25) (layer "F.Cu") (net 23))
 (segment (start 61.236796 73.164563) (end 61.987907 73.915674) (width 0.25) (layer "F.Cu") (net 23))
 (segment (start 62.2808 74.622781) (end 62.2808 83.898159) (width 0.25) (layer "F.Cu") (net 23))
 (arc (start 62.2808 83.898159) (mid 62.509162 85.04621) (end 63.15948 86.01948) (width 0.25) (layer "F.Cu") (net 23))
 (arc (start 62.2808 74.622781) (mid 62.20468 74.240098) (end 61.987907 73.915674) (width 0.25) (layer "F.Cu") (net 23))
 (segment (start 63.64208 83.96208) (end 66.04 86.36) (width 0.25) (layer "F.Cu") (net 24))
 (segment (start 62.7634 74.605381) (end 62.7634 81.840759) (width 0.25) (layer "F.Cu") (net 24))
 (segment (start 61.590349 72.81101) (end 62.32406 73.544721) (width 0.25) (layer "F.Cu") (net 24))
 (arc (start 62.32406 73.544721) (mid 62.649219 74.031356) (end 62.7634 74.605381) (width 0.25) (layer "F.Cu") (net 24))
 (arc (start 62.7634 81.840759) (mid 62.991762 82.98881) (end 63.64208 83.96208) (width 0.25) (layer "F.Cu") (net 24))
 (segment (start 61.943903 72.457456) (end 62.660214 73.173767) (width 0.25) (layer "F.Cu") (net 25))
 (segment (start 64.12468 81.90468) (end 66.04 83.82) (width 0.25) (layer "F.Cu") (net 25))
 (segment (start 63.246 74.58798) (end 63.246 79.783359) (width 0.25) (layer "F.Cu") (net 25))
 (arc (start 64.12468 81.90468) (mid 63.474361 80.93141) (end 63.246 79.783359) (width 0.25) (layer "F.Cu") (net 25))
 (arc (start 63.246 74.58798) (mid 63.093759 73.822613) (end 62.660214 73.173767) (width 0.25) (layer "F.Cu") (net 25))
 (segment (start 63.7286 74.570581) (end 63.7286 77.725959) (width 0.25) (layer "F.Cu") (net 26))
 (segment (start 62.297456 72.103903) (end 62.996367 72.802814) (width 0.25) (layer "F.Cu") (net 26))
 (segment (start 64.60728 79.84728) (end 66.04 81.28) (width 0.25) (layer "F.Cu") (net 26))
 (arc (start 63.7286 74.570581) (mid 63.538299 73.613872) (end 62.996367 72.802814) (width 0.25) (layer "F.Cu") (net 26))
 (arc (start 63.7286 77.725959) (mid 63.956962 78.87401) (end 64.60728 79.84728) (width 0.25) (layer "F.Cu") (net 26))
 (segment (start 64.2112 76.037647) (end 64.2112 74.55318) (width 0.25) (layer "F.Cu") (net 27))
 (segment (start 66.04 78.74) (end 64.828895 77.528895) (width 0.25) (layer "F.Cu") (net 27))
 (segment (start 63.33252 72.431859) (end 62.65101 71.750349) (width 0.25) (layer "F.Cu") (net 27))
 (arc (start 64.2112 74.55318) (mid 63.982838 73.405129) (end 63.33252 72.431859) (width 0.25) (layer "F.Cu") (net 27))
 (arc (start 64.2112 76.037647) (mid 64.371734 76.844705) (end 64.828895 77.528895) (width 0.25) (layer "F.Cu") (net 27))
 (segment (start 63.004563 71.396796) (end 63.668674 72.060907) (width 0.25) (layer "F.Cu") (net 28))
 (segment (start 65.571236 75.889224) (end 65.048149 75.366137) (width 0.25) (layer "F.Cu") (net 28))
 (arc (start 64.6938 74.53578) (mid 64.427378 73.196388) (end 63.668674 72.060907) (width 0.25) (layer "F.Cu") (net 28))
 (arc (start 64.692557 74.507662) (mid 64.784972 74.972265) (end 65.048149 75.366137) (width 0.25) (layer "F.Cu") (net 28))
 (segment (start 63.358116 71.043243) (end 65.974873 73.66) (width 0.25) (layer "F.Cu") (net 29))
 (segment (start 66.04 73.66) (end 65.974873 73.66) (width 0.25) (layer "F.Cu") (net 29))
 (segment (start 65.532 71.628) (end 66.04 71.12) (width 0.25) (layer "F.Cu") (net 30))
 (segment (start 64.985253 71.628) (end 65.532 71.628) (width 0.25) (layer "F.Cu") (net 30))
 (segment (start 65.581044 71.440687) (end 65.553552 71.468177) (width 0.25) (layer "F.Cu") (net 30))
 (segment (start 63.71167 70.689689) (end 64.412908 71.390927) (width 0.25) (layer "F.Cu") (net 30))
 (arc (start 65.495549 71.466953) (mid 65.317151 71.586146) (end 65.10672 71.628) (width 0.25) (layer "F.Cu") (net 30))
 (arc (start 64.985253 71.628) (mid 64.675502 71.566387) (end 64.412908 71.390927) (width 0.25) (layer "F.Cu") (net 30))
 (segment (start 65.532 68.072) (end 66.04 68.58) (width 0.25) (layer "F.Cu") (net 31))
 (segment (start 64.985253 68.072) (end 65.532 68.072) (width 0.25) (layer "F.Cu") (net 31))
 (segment (start 63.71167 69.010311) (end 64.412908 68.309073) (width 0.25) (layer "F.Cu") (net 31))
 (segment (start 65.581044 68.259313) (end 65.553552 68.231823) (width 0.25) (layer "F.Cu") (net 31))
 (arc (start 64.985253 68.072) (mid 64.675502 68.133613) (end 64.412908 68.309073) (width 0.25) (layer "F.Cu") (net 31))
 (arc (start 65.495549 68.233047) (mid 65.317151 68.113854) (end 65.10672 68.072) (width 0.25) (layer "F.Cu") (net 31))
 (segment (start 66.04 66.04) (end 65.974873 66.04) (width 0.25) (layer "F.Cu") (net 32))
 (segment (start 63.358116 68.656757) (end 65.974873 66.04) (width 0.25) (layer "F.Cu") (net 32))
 (segment (start 63.004563 68.303204) (end 63.668674 67.639093) (width 0.25) (layer "F.Cu") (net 33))
 (segment (start 65.571236 63.810776) (end 65.048149 64.333863) (width 0.25) (layer "F.Cu") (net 33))
 (arc (start 64.692557 65.192338) (mid 64.784972 64.727735) (end 65.048149 64.333863) (width 0.25) (layer "F.Cu") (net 33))
 (arc (start 64.6938 65.16422) (mid 64.427378 66.503612) (end 63.668674 67.639093) (width 0.25) (layer "F.Cu") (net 33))
 (segment (start 63.33252 67.268141) (end 62.65101 67.949651) (width 0.25) (layer "F.Cu") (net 34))
 (segment (start 66.04 60.96) (end 64.828895 62.171105) (width 0.25) (layer "F.Cu") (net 34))
 (segment (start 64.2112 63.662353) (end 64.2112 65.14682) (width 0.25) (layer "F.Cu") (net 34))
 (arc (start 64.2112 63.662353) (mid 64.371734 62.855295) (end 64.828895 62.171105) (width 0.25) (layer "F.Cu") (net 34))
 (arc (start 64.2112 65.14682) (mid 63.982838 66.294871) (end 63.33252 67.268141) (width 0.25) (layer "F.Cu") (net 34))
 (segment (start 62.297456 67.596097) (end 62.996367 66.897186) (width 0.25) (layer "F.Cu") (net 35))
 (segment (start 63.7286 65.129419) (end 63.7286 61.974041) (width 0.25) (layer "F.Cu") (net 35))
 (segment (start 64.60728 59.85272) (end 66.04 58.42) (width 0.25) (layer "F.Cu") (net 35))
 (arc (start 63.7286 61.974041) (mid 63.956962 60.82599) (end 64.60728 59.85272) (width 0.25) (layer "F.Cu") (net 35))
 (arc (start 63.7286 65.129419) (mid 63.538299 66.086128) (end 62.996367 66.897186) (width 0.25) (layer "F.Cu") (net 35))
 (segment (start 64.12468 57.79532) (end 66.04 55.88) (width 0.25) (layer "F.Cu") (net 36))
 (segment (start 61.943903 67.242544) (end 62.660214 66.526233) (width 0.25) (layer "F.Cu") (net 36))
 (segment (start 63.246 65.11202) (end 63.246 59.916641) (width 0.25) (layer "F.Cu") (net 36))
 (arc (start 64.12468 57.79532) (mid 63.474361 58.76859) (end 63.246 59.916641) (width 0.25) (layer "F.Cu") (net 36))
 (arc (start 63.246 65.11202) (mid 63.093759 65.877387) (end 62.660214 66.526233) (width 0.25) (layer "F.Cu") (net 36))
 (segment (start 63.64208 55.73792) (end 66.04 53.34) (width 0.25) (layer "F.Cu") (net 37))
 (segment (start 62.7634 65.094619) (end 62.7634 57.859241) (width 0.25) (layer "F.Cu") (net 37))
 (segment (start 61.590349 66.88899) (end 62.32406 66.155279) (width 0.25) (layer "F.Cu") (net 37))
 (arc (start 62.7634 57.859241) (mid 62.991762 56.71119) (end 63.64208 55.73792) (width 0.25) (layer "F.Cu") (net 37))
 (arc (start 62.32406 66.155279) (mid 62.649219 65.668644) (end 62.7634 65.094619) (width 0.25) (layer "F.Cu") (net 37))
 (segment (start 62.2808 65.077219) (end 62.2808 55.801841) (width 0.25) (layer "F.Cu") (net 38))
 (segment (start 61.236796 66.535437) (end 61.987907 65.784326) (width 0.25) (layer "F.Cu") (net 38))
 (segment (start 63.15948 53.68052) (end 66.04 50.8) (width 0.25) (layer "F.Cu") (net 38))
 (arc (start 62.2808 65.077219) (mid 62.20468 65.459902) (end 61.987907 65.784326) (width 0.25) (layer "F.Cu") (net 38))
 (arc (start 62.2808 55.801841) (mid 62.509162 54.65379) (end 63.15948 53.68052) (width 0.25) (layer "F.Cu") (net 38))
 (segment (start 61.7982 65.05982) (end 61.7982 53.744441) (width 0.25) (layer "F.Cu") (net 39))
 (segment (start 62.67688 51.62312) (end 66.04 48.26) (width 0.25) (layer "F.Cu") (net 39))
 (segment (start 60.883243 66.181884) (end 61.651754 65.413373) (width 0.25) (layer "F.Cu") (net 39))
 (arc (start 61.7982 53.744441) (mid 62.026562 52.59639) (end 62.67688 51.62312) (width 0.25) (layer "F.Cu") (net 39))
 (arc (start 61.7982 65.05982) (mid 61.76014 65.251161) (end 61.651754 65.413373) (width 0.25) (layer "F.Cu") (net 39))
 (segment (start 61.308 65.01448) (end 61.308 51.694641) (width 0.25) (layer "F.Cu") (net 40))
 (segment (start 62.18668 49.57332) (end 66.04 45.72) (width 0.25) (layer "F.Cu") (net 40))
 (segment (start 60.529689 65.82833) (end 61.28287 65.075149) (width 0.25) (layer "F.Cu") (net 40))
 (arc (start 61.308 65.01448) (mid 61.301469 65.047314) (end 61.28287 65.075149) (width 0.25) (layer "F.Cu") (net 40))
 (arc (start 61.308 51.694641) (mid 61.536362 50.54659) (end 62.18668 49.57332) (width 0.25) (layer "F.Cu") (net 40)))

